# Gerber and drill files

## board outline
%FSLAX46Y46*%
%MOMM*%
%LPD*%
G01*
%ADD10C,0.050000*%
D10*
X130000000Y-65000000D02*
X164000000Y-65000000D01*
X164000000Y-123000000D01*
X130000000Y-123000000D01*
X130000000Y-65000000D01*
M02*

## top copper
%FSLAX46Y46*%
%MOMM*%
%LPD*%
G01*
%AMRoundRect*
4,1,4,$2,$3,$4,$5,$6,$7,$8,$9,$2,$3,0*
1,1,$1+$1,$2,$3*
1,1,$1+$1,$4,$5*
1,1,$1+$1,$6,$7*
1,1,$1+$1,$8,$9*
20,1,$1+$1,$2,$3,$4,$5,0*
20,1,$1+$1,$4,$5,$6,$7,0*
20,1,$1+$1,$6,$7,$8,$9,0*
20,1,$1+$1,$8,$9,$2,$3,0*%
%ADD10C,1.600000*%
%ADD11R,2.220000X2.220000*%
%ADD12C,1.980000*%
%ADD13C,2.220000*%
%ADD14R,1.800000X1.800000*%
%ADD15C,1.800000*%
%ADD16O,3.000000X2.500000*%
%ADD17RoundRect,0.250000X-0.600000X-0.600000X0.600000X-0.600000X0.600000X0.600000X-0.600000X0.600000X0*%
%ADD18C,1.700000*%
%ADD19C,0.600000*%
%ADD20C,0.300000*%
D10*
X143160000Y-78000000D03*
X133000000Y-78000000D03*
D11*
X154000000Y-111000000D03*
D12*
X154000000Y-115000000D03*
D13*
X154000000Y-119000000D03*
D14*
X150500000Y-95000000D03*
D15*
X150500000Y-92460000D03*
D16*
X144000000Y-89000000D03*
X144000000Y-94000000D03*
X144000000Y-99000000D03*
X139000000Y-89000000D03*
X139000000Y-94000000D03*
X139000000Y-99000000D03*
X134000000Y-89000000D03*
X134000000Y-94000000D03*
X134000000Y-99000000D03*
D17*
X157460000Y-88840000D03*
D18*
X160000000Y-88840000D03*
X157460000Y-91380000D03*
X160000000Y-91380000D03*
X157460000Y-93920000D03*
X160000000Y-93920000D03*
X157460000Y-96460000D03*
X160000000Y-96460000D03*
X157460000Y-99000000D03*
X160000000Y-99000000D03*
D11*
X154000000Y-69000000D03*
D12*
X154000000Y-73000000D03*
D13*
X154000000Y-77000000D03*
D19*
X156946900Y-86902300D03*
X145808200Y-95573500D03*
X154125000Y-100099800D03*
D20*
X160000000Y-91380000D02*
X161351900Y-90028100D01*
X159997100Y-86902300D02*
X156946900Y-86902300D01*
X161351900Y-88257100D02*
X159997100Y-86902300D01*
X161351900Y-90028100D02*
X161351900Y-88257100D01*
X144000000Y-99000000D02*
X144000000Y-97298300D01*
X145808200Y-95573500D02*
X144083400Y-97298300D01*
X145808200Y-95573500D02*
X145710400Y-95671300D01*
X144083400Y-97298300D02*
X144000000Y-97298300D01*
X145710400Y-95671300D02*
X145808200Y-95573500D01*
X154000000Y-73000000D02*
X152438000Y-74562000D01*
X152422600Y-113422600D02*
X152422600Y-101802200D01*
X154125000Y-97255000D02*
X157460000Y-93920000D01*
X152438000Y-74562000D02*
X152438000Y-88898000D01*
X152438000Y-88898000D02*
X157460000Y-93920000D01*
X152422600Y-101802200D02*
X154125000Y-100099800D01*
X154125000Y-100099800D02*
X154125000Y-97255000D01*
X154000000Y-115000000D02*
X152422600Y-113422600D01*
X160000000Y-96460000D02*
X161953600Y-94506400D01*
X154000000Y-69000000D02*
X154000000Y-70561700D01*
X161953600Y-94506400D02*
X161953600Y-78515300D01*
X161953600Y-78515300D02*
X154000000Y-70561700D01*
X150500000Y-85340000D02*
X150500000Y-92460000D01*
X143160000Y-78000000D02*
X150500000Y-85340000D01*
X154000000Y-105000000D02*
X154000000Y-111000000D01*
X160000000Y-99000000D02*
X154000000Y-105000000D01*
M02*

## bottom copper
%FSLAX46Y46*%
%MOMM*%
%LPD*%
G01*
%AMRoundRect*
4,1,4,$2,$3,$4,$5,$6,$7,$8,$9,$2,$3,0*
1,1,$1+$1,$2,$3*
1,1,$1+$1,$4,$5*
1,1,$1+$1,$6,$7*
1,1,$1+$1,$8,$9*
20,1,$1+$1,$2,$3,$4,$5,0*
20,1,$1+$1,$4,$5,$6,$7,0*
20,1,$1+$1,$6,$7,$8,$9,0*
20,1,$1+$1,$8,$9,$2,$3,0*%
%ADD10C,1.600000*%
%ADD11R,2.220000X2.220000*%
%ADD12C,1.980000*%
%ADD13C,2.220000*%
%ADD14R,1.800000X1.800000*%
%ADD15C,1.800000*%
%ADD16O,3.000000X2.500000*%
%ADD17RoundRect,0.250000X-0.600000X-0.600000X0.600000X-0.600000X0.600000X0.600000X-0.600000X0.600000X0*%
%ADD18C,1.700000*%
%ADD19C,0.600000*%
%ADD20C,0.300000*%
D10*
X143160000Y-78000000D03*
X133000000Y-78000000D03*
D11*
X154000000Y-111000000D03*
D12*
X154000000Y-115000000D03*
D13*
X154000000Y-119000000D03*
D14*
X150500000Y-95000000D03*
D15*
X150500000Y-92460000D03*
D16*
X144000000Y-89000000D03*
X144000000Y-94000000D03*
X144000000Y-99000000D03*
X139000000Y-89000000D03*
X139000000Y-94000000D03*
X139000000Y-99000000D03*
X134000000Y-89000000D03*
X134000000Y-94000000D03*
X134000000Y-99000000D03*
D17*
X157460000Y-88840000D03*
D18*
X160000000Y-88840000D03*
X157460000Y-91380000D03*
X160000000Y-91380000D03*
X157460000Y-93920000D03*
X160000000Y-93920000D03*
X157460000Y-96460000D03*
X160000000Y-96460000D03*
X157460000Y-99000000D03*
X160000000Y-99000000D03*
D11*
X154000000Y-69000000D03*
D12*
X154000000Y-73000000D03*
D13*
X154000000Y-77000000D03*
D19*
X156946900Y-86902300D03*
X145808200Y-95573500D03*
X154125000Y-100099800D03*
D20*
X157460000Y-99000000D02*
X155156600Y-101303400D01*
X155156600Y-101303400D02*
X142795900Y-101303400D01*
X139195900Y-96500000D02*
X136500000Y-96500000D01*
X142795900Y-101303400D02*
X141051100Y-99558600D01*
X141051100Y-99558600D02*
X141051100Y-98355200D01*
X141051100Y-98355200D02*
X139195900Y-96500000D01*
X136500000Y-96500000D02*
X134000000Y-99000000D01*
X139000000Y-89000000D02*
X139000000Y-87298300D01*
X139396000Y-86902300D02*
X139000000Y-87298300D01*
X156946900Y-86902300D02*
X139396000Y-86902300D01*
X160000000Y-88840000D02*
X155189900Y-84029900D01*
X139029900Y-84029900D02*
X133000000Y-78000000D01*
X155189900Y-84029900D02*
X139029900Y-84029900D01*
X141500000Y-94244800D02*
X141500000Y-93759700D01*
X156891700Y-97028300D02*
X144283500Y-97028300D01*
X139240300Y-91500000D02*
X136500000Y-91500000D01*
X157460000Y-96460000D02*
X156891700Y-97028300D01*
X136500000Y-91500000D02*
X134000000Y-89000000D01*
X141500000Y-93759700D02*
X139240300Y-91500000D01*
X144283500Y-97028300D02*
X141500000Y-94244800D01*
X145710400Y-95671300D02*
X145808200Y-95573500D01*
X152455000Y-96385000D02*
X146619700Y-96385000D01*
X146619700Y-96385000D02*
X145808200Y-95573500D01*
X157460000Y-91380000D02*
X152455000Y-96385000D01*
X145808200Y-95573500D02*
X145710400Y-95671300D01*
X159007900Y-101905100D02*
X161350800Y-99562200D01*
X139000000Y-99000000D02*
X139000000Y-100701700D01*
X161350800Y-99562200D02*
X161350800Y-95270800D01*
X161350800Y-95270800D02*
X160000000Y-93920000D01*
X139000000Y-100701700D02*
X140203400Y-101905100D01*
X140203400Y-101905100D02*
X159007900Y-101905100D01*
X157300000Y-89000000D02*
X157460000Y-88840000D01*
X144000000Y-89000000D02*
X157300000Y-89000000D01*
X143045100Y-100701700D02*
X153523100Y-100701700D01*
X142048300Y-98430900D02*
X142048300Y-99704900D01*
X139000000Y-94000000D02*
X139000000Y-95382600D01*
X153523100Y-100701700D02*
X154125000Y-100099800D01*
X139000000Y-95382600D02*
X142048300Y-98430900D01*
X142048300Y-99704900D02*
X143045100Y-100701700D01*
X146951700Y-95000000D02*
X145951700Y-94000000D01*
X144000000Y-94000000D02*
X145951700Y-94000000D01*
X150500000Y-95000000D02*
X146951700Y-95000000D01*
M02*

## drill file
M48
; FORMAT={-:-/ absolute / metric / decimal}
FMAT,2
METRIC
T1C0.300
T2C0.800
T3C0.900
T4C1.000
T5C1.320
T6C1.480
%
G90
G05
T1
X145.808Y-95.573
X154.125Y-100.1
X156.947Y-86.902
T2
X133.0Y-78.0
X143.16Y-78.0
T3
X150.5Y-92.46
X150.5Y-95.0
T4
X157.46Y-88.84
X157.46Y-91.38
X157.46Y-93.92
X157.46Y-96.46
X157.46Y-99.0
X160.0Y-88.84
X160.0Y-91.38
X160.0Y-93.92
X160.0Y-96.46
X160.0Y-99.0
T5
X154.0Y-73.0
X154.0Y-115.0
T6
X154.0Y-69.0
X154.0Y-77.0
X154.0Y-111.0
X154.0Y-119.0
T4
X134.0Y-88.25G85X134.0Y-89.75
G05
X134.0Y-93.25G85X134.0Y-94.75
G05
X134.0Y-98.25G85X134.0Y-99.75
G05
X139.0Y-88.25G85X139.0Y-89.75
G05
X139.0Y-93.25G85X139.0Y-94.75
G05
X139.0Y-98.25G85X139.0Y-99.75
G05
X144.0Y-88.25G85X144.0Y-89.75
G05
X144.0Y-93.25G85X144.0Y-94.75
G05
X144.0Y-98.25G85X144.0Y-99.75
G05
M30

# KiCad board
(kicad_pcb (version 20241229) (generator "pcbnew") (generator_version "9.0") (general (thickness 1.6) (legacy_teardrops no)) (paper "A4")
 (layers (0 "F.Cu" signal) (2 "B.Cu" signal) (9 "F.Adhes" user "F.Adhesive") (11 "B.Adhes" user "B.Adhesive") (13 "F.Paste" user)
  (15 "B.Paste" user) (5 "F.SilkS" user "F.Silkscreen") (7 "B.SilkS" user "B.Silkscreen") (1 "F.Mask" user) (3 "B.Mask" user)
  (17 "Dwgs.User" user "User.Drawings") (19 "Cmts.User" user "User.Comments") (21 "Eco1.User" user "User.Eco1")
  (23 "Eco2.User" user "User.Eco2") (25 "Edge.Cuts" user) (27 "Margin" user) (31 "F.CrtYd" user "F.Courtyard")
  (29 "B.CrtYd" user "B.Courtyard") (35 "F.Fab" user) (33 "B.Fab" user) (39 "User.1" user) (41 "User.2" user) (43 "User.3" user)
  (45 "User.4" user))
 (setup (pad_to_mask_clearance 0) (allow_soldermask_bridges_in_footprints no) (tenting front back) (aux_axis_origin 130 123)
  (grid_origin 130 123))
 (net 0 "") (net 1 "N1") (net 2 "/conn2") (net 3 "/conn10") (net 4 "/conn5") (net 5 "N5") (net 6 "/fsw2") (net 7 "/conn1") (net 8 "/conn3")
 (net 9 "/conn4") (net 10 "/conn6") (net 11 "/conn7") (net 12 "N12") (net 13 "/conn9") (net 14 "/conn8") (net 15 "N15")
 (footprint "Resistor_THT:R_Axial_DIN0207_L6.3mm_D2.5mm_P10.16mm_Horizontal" (layer "F.Cu") (at 143.16 78 180)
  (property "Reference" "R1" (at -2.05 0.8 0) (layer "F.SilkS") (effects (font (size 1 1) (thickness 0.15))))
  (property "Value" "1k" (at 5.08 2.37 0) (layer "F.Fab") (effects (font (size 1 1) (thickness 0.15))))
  (pad "1" thru_hole circle (at 0 0 180) (size 1.6 1.6) (drill 0.8) (layers "*.Cu" "*.Mask") (remove_unused_layers no) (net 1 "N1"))
  (pad "2" thru_hole circle (at 10.16 0 180) (size 1.6 1.6) (drill 0.8) (layers "*.Cu" "*.Mask") (remove_unused_layers no) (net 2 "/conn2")))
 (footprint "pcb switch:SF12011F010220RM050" (layer "F.Cu") (at 154 111 -90)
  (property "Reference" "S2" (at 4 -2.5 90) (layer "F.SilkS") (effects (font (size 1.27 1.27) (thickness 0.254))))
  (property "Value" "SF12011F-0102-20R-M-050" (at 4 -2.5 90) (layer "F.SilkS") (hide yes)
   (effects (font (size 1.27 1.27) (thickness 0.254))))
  (pad "1" thru_hole rect (at 0 0 270) (size 2.22 2.22) (drill 1.48) (layers "*.Cu" "*.Mask") (remove_unused_layers no) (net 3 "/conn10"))
  (pad "2" thru_hole circle (at 4 0 270) (size 1.98 1.98) (drill 1.32) (layers "*.Cu" "*.Mask") (remove_unused_layers no) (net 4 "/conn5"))
  (pad "3" thru_hole circle (at 8 0 270) (size 2.22 2.22) (drill 1.48) (layers "*.Cu" "*.Mask") (remove_unused_layers no) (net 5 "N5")))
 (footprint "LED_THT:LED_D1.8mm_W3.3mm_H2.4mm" (layer "F.Cu") (at 150.5 95 90)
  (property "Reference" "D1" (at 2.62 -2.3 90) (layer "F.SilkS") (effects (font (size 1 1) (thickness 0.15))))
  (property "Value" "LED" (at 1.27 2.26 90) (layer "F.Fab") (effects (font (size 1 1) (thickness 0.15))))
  (pad "1" thru_hole rect (at 0 0 90) (size 1.8 1.8) (drill 0.9) (layers "*.Cu" "*.Mask") (remove_unused_layers no) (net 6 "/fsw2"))
  (pad "2" thru_hole circle (at 2.54 0 90) (size 1.8 1.8) (drill 0.9) (layers "*.Cu" "*.Mask") (remove_unused_layers no) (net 1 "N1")))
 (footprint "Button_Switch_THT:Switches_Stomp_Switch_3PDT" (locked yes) (layer "F.Cu") (at 139 94 -90)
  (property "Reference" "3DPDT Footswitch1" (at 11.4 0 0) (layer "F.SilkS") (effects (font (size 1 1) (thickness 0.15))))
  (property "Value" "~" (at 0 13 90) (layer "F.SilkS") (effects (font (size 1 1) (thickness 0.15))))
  (pad "1" thru_hole oval (at -5 -5 270) (size 2.5 3) (drill oval 2.5 1) (layers "*.Cu" "*.Mask" "F.SilkS") (remove_unused_layers no)
   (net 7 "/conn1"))
  (pad "2" thru_hole oval (at 0 -5 270) (size 2.5 3) (drill oval 2.5 1) (layers "*.Cu" "*.Mask" "F.SilkS") (remove_unused_layers no)
   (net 6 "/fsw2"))
  (pad "3" thru_hole oval (at 5 -5 270) (size 2.5 3) (drill oval 2.5 1) (layers "*.Cu" "*.Mask" "F.SilkS") (remove_unused_layers no)
   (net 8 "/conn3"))
  (pad "4" thru_hole oval (at -5 0 270) (size 2.5 3) (drill oval 2.5 1) (layers "*.Cu" "*.Mask" "F.SilkS") (remove_unused_layers no)
   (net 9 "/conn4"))
  (pad "5" thru_hole oval (at 0 0 270) (size 2.5 3) (drill oval 2.5 1) (layers "*.Cu" "*.Mask" "F.SilkS") (remove_unused_layers no)
   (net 4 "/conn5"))
  (pad "6" thru_hole oval (at 5 0 270) (size 2.5 3) (drill oval 2.5 1) (layers "*.Cu" "*.Mask" "F.SilkS") (remove_unused_layers no)
   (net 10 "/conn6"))
  (pad "7" thru_hole oval (at -5 5 270) (size 2.5 3) (drill oval 2.5 1) (layers "*.Cu" "*.Mask" "F.SilkS") (remove_unused_layers no)
   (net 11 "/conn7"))
  (pad "8" thru_hole oval (at 0 5 270) (size 2.5 3) (drill oval 2.5 1) (layers "*.Cu" "*.Mask" "F.SilkS") (remove_unused_layers no)
   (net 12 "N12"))
  (pad "9" thru_hole oval (at 5 5 270) (size 2.5 3) (drill oval 2.5 1) (layers "*.Cu" "*.Mask" "F.SilkS") (remove_unused_layers no)
   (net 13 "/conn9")))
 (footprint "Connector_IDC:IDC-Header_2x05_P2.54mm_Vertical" (layer "F.Cu") (at 157.46 88.84)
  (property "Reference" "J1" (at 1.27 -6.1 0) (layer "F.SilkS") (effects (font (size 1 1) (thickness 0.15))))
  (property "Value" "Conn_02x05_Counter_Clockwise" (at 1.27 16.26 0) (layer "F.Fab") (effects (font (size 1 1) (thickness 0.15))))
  (pad "1" thru_hole roundrect (at 0 0) (size 1.7 1.7) (drill 1) (layers "*.Cu" "*.Mask") (remove_unused_layers no)
   (roundrect_rratio 0.147059) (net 7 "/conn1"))
  (pad "2" thru_hole circle (at 2.54 0) (size 1.7 1.7) (drill 1) (layers "*.Cu" "*.Mask") (remove_unused_layers no) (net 2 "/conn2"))
  (pad "3" thru_hole circle (at 0 2.54) (size 1.7 1.7) (drill 1) (layers "*.Cu" "*.Mask") (remove_unused_layers no) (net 8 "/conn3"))
  (pad "4" thru_hole circle (at 2.54 2.54) (size 1.7 1.7) (drill 1) (layers "*.Cu" "*.Mask") (remove_unused_layers no) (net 9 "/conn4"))
  (pad "5" thru_hole circle (at 0 5.08) (size 1.7 1.7) (drill 1) (layers "*.Cu" "*.Mask") (remove_unused_layers no) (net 4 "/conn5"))
  (pad "6" thru_hole circle (at 2.54 5.08) (size 1.7 1.7) (drill 1) (layers "*.Cu" "*.Mask") (remove_unused_layers no) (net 10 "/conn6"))
  (pad "7" thru_hole circle (at 0 7.62) (size 1.7 1.7) (drill 1) (layers "*.Cu" "*.Mask") (remove_unused_layers no) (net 11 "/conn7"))
  (pad "8" thru_hole circle (at 2.54 7.62) (size 1.7 1.7) (drill 1) (layers "*.Cu" "*.Mask") (remove_unused_layers no) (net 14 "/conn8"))
  (pad "9" thru_hole circle (at 0 10.16) (size 1.7 1.7) (drill 1) (layers "*.Cu" "*.Mask") (remove_unused_layers no) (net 13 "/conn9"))
  (pad "10" thru_hole circle (at 2.54 10.16) (size 1.7 1.7) (drill 1) (layers "*.Cu" "*.Mask") (remove_unused_layers no) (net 3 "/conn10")))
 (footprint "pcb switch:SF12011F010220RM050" (layer "F.Cu") (at 154 69 -90)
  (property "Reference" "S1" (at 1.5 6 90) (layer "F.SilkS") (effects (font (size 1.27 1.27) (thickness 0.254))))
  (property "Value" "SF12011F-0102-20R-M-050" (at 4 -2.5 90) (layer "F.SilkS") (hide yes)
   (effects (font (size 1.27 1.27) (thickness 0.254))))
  (pad "1" thru_hole rect (at 0 0 270) (size 2.22 2.22) (drill 1.48) (layers "*.Cu" "*.Mask") (remove_unused_layers no) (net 14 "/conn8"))
  (pad "2" thru_hole circle (at 4 0 270) (size 1.98 1.98) (drill 1.32) (layers "*.Cu" "*.Mask") (remove_unused_layers no) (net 4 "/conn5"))
  (pad "3" thru_hole circle (at 8 0 270) (size 2.22 2.22) (drill 1.48) (layers "*.Cu" "*.Mask") (remove_unused_layers no) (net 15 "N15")))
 (gr_rect (start 130 65) (end 164 123) (stroke (width 0.05) (type solid)) (fill no) (layer "Edge.Cuts"))
 (segment (start 157.46 99) (end 155.1566 101.3034) (width 0.3) (layer "B.Cu") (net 13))
 (segment (start 155.1566 101.3034) (end 142.7959 101.3034) (width 0.3) (layer "B.Cu") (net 13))
 (segment (start 139.1959 96.5) (end 136.5 96.5) (width 0.3) (layer "B.Cu") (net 13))
 (segment (start 142.7959 101.3034) (end 141.0511 99.5586) (width 0.3) (layer "B.Cu") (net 13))
 (segment (start 141.0511 99.5586) (end 141.0511 98.3552) (width 0.3) (layer "B.Cu") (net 13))
 (segment (start 141.0511 98.3552) (end 139.1959 96.5) (width 0.3) (layer "B.Cu") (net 13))
 (segment (start 136.5 96.5) (end 134 99) (width 0.3) (layer "B.Cu") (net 13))
 (segment (start 160 91.38) (end 161.3519 90.0281) (width 0.3) (layer "F.Cu") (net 9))
 (segment (start 159.9971 86.9023) (end 156.9469 86.9023) (width 0.3) (layer "F.Cu") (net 9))
 (segment (start 161.3519 88.2571) (end 159.9971 86.9023) (width 0.3) (layer "F.Cu") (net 9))
 (segment (start 161.3519 90.0281) (end 161.3519 88.2571) (width 0.3) (layer "F.Cu") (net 9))
 (via (at 156.9469 86.9023) (size 0.6) (drill 0.3) (layers "F.Cu" "B.Cu") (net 9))
 (segment (start 139 89) (end 139 87.2983) (width 0.3) (layer "B.Cu") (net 9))
 (segment (start 139.396 86.9023) (end 139 87.2983) (width 0.3) (layer "B.Cu") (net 9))
 (segment (start 156.9469 86.9023) (end 139.396 86.9023) (width 0.3) (layer "B.Cu") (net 9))
 (segment (start 160 88.84) (end 155.1899 84.0299) (width 0.3) (layer "B.Cu") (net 2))
 (segment (start 139.0299 84.0299) (end 133 78) (width 0.3) (layer "B.Cu") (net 2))
 (segment (start 155.1899 84.0299) (end 139.0299 84.0299) (width 0.3) (layer "B.Cu") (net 2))
 (segment (start 141.5 94.2448) (end 141.5 93.7597) (width 0.3) (layer "B.Cu") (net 11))
 (segment (start 156.8917 97.0283) (end 144.2835 97.0283) (width 0.3) (layer "B.Cu") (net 11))
 (segment (start 139.2403 91.5) (end 136.5 91.5) (width 0.3) (layer "B.Cu") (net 11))
 (segment (start 157.46 96.46) (end 156.8917 97.0283) (width 0.3) (layer "B.Cu") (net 11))
 (segment (start 136.5 91.5) (end 134 89) (width 0.3) (layer "B.Cu") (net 11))
 (segment (start 141.5 93.7597) (end 139.2403 91.5) (width 0.3) (layer "B.Cu") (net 11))
 (segment (start 144.2835 97.0283) (end 141.5 94.2448) (width 0.3) (layer "B.Cu") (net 11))
 (segment (start 144 99) (end 144 97.2983) (width 0.3) (layer "F.Cu") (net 8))
 (segment (start 145.8082 95.5735) (end 144.0834 97.2983) (width 0.3) (layer "F.Cu") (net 8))
 (segment (start 145.8082 95.5735) (end 145.7104 95.6713) (width 0.3) (layer "F.Cu") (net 8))
 (segment (start 144.0834 97.2983) (end 144 97.2983) (width 0.3) (layer "F.Cu") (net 8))
 (segment (start 145.7104 95.6713) (end 145.8082 95.5735) (width 0.3) (layer "F.Cu") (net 8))
 (via (at 145.8082 95.5735) (size 0.6) (drill 0.3) (layers "F.Cu" "B.Cu") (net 8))
 (segment (start 145.7104 95.6713) (end 145.8082 95.5735) (width 0.3) (layer "B.Cu") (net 8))
 (segment (start 152.455 96.385) (end 146.6197 96.385) (width 0.3) (layer "B.Cu") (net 8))
 (segment (start 146.6197 96.385) (end 145.8082 95.5735) (width 0.3) (layer "B.Cu") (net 8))
 (segment (start 157.46 91.38) (end 152.455 96.385) (width 0.3) (layer "B.Cu") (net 8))
 (segment (start 145.8082 95.5735) (end 145.7104 95.6713) (width 0.3) (layer "B.Cu") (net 8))
 (segment (start 159.0079 101.9051) (end 161.3508 99.5622) (width 0.3) (layer "B.Cu") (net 10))
 (segment (start 139 99) (end 139 100.7017) (width 0.3) (layer "B.Cu") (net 10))
 (segment (start 161.3508 99.5622) (end 161.3508 95.2708) (width 0.3) (layer "B.Cu") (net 10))
 (segment (start 161.3508 95.2708) (end 160 93.92) (width 0.3) (layer "B.Cu") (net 10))
 (segment (start 139 100.7017) (end 140.2034 101.9051) (width 0.3) (layer "B.Cu") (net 10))
 (segment (start 140.2034 101.9051) (end 159.0079 101.9051) (width 0.3) (layer "B.Cu") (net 10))
 (segment (start 157.3 89) (end 157.46 88.84) (width 0.3) (layer "B.Cu") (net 7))
 (segment (start 144 89) (end 157.3 89) (width 0.3) (layer "B.Cu") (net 7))
 (segment (start 154 73) (end 152.438 74.562) (width 0.3) (layer "F.Cu") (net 4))
 (segment (start 152.4226 113.4226) (end 152.4226 101.8022) (width 0.3) (layer "F.Cu") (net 4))
 (segment (start 154.125 97.255) (end 157.46 93.92) (width 0.3) (layer "F.Cu") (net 4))
 (segment (start 152.438 74.562) (end 152.438 88.898) (width 0.3) (layer "F.Cu") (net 4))
 (segment (start 152.438 88.898) (end 157.46 93.92) (width 0.3) (layer "F.Cu") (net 4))
 (segment (start 152.4226 101.8022) (end 154.125 100.0998) (width 0.3) (layer "F.Cu") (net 4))
 (segment (start 154.125 100.0998) (end 154.125 97.255) (width 0.3) (layer "F.Cu") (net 4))
 (segment (start 154 115) (end 152.4226 113.4226) (width 0.3) (layer "F.Cu") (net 4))
 (via (at 154.125 100.0998) (size 0.6) (drill 0.3) (layers "F.Cu" "B.Cu") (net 4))
 (segment (start 143.0451 100.7017) (end 153.5231 100.7017) (width 0.3) (layer "B.Cu") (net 4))
 (segment (start 142.0483 98.4309) (end 142.0483 99.7049) (width 0.3) (layer "B.Cu") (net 4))
 (segment (start 139 94) (end 139 95.3826) (width 0.3) (layer "B.Cu") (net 4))
 (segment (start 153.5231 100.7017) (end 154.125 100.0998) (width 0.3) (layer "B.Cu") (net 4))
 (segment (start 139 95.3826) (end 142.0483 98.4309) (width 0.3) (layer "B.Cu") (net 4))
 (segment (start 142.0483 99.7049) (end 143.0451 100.7017) (width 0.3) (layer "B.Cu") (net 4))
 (segment (start 160 96.46) (end 161.9536 94.5064) (width 0.3) (layer "F.Cu") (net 14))
 (segment (start 154 69) (end 154 70.5617) (width 0.3) (layer "F.Cu") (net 14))
 (segment (start 161.9536 94.5064) (end 161.9536 78.5153) (width 0.3) (layer "F.Cu") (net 14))
 (segment (start 161.9536 78.5153) (end 154 70.5617) (width 0.3) (layer "F.Cu") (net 14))
 (segment (start 150.5 85.34) (end 150.5 92.46) (width 0.3) (layer "F.Cu") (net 1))
 (segment (start 143.16 78) (end 150.5 85.34) (width 0.3) (layer "F.Cu") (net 1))
 (segment (start 146.9517 95) (end 145.9517 94) (width 0.3) (layer "B.Cu") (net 6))
 (segment (start 144 94) (end 145.9517 94) (width 0.3) (layer "B.Cu") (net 6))
 (segment (start 150.5 95) (end 146.9517 95) (width 0.3) (layer "B.Cu") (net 6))
 (segment (start 154 105) (end 154 111) (width 0.3) (layer "F.Cu") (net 3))
 (segment (start 160 99) (end 154 105) (width 0.3) (layer "F.Cu") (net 3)))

